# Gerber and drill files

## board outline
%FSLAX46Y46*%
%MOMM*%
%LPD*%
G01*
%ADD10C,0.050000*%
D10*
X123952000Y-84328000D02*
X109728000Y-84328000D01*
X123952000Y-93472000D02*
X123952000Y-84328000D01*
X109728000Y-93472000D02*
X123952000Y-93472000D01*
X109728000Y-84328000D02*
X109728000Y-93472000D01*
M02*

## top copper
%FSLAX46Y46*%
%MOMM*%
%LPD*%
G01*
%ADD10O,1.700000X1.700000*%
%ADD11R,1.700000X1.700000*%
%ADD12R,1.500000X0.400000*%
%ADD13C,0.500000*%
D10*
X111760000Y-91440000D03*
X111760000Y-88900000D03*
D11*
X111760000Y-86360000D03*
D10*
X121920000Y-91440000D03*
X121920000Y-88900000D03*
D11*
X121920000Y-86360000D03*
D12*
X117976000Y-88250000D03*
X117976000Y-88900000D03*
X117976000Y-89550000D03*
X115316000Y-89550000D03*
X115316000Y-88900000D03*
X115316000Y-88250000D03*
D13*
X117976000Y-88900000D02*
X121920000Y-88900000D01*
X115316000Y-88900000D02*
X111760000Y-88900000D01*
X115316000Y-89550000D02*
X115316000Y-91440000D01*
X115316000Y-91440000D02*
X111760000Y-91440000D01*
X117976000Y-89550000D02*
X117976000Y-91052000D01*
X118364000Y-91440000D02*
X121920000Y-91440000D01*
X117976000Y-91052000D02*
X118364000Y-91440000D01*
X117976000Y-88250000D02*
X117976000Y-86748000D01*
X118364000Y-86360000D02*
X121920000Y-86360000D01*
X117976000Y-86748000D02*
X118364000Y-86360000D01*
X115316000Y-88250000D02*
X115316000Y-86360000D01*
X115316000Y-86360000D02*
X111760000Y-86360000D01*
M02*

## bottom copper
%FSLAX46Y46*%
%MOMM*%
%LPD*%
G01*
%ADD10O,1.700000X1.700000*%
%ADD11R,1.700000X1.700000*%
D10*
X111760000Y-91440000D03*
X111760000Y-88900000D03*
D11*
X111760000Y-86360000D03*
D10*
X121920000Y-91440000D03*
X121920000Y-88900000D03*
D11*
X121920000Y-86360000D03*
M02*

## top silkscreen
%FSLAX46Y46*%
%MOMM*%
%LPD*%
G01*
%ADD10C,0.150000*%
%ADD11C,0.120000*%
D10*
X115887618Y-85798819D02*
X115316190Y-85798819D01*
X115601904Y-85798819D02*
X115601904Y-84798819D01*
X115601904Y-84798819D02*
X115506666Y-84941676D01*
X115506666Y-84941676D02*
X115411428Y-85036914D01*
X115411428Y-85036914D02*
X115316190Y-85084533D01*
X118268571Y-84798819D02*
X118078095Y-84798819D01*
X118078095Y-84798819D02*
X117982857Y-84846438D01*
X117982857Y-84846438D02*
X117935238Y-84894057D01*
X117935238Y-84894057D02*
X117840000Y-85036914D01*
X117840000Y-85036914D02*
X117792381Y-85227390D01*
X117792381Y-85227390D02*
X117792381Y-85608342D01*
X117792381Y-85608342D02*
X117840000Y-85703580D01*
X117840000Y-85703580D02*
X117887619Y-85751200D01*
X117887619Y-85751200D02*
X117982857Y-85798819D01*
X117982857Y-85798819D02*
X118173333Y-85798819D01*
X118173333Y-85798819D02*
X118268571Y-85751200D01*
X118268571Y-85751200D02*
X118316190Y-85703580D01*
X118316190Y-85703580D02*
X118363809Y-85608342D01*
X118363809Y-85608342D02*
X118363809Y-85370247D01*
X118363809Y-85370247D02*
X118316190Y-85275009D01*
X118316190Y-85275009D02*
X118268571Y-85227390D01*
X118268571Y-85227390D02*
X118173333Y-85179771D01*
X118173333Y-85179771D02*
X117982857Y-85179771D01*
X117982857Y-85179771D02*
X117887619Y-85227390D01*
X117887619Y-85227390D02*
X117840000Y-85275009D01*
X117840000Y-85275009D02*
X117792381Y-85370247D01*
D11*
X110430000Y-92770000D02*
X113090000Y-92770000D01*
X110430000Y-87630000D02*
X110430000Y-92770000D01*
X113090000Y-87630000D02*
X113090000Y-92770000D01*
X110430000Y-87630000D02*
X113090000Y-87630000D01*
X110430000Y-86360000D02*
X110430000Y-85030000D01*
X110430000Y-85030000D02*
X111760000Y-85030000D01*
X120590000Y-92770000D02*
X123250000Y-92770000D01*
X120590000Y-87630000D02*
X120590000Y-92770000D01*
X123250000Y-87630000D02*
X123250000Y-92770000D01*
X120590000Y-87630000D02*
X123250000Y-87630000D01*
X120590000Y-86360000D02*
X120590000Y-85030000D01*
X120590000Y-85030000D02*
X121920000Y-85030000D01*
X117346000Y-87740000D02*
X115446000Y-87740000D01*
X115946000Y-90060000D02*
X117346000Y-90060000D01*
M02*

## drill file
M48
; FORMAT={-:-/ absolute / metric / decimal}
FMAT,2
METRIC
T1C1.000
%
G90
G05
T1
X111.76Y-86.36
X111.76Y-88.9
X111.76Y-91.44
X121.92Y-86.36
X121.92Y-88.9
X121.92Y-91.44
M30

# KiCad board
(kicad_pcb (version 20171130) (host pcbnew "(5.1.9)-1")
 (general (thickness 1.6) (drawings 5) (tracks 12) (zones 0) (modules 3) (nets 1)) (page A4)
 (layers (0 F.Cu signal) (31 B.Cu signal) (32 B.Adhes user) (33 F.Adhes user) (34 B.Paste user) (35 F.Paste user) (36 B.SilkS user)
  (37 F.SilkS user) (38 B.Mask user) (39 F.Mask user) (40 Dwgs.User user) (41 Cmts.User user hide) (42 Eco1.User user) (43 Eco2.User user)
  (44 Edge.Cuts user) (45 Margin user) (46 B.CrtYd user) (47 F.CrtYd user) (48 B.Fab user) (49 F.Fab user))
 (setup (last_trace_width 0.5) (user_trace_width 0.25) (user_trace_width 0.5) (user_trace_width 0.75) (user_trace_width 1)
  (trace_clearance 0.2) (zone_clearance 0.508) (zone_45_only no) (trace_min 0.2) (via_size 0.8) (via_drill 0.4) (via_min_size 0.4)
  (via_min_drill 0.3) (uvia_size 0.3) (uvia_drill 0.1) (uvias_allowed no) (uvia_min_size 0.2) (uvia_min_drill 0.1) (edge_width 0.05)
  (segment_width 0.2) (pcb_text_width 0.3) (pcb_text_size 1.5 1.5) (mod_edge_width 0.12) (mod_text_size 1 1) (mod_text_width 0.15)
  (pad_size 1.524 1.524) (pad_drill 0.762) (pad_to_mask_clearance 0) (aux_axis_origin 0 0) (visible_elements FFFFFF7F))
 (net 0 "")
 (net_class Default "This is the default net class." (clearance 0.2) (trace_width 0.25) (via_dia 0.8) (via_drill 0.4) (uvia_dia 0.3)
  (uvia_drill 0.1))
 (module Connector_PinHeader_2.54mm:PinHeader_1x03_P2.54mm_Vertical (layer F.Cu) (at 111.76 86.36)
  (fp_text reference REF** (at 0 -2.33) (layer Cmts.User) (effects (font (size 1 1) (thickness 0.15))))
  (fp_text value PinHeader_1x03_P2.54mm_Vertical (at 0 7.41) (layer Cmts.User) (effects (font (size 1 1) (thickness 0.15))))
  (fp_line (start -1.33 6.41) (end 1.33 6.41) (layer F.SilkS) (width 0.12))
  (fp_line (start -1.33 1.27) (end -1.33 6.41) (layer F.SilkS) (width 0.12))
  (fp_line (start 1.33 1.27) (end 1.33 6.41) (layer F.SilkS) (width 0.12))
  (fp_line (start -1.33 1.27) (end 1.33 1.27) (layer F.SilkS) (width 0.12))
  (fp_line (start -1.33 0) (end -1.33 -1.33) (layer F.SilkS) (width 0.12))
  (fp_line (start -1.33 -1.33) (end 0 -1.33) (layer F.SilkS) (width 0.12))
  (pad 3 thru_hole oval (at 0 5.08) (size 1.7 1.7) (drill 1) (layers *.Cu *.Mask))
  (pad 2 thru_hole oval (at 0 2.54) (size 1.7 1.7) (drill 1) (layers *.Cu *.Mask))
  (pad 1 thru_hole rect (at 0 0) (size 1.7 1.7) (drill 1) (layers *.Cu *.Mask)))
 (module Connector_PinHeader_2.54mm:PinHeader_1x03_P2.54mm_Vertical (layer F.Cu) (at 121.92 86.36)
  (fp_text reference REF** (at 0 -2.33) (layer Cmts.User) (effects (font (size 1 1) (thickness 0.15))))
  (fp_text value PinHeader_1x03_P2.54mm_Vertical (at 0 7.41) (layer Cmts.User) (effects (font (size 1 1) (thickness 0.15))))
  (fp_line (start -1.33 6.41) (end 1.33 6.41) (layer F.SilkS) (width 0.12))
  (fp_line (start -1.33 1.27) (end -1.33 6.41) (layer F.SilkS) (width 0.12))
  (fp_line (start 1.33 1.27) (end 1.33 6.41) (layer F.SilkS) (width 0.12))
  (fp_line (start -1.33 1.27) (end 1.33 1.27) (layer F.SilkS) (width 0.12))
  (fp_line (start -1.33 0) (end -1.33 -1.33) (layer F.SilkS) (width 0.12))
  (fp_line (start -1.33 -1.33) (end 0 -1.33) (layer F.SilkS) (width 0.12))
  (pad 3 thru_hole oval (at 0 5.08) (size 1.7 1.7) (drill 1) (layers *.Cu *.Mask))
  (pad 2 thru_hole oval (at 0 2.54) (size 1.7 1.7) (drill 1) (layers *.Cu *.Mask))
  (pad 1 thru_hole rect (at 0 0) (size 1.7 1.7) (drill 1) (layers *.Cu *.Mask)))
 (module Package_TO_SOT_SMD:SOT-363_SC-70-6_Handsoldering (layer F.Cu) (at 116.646 88.9)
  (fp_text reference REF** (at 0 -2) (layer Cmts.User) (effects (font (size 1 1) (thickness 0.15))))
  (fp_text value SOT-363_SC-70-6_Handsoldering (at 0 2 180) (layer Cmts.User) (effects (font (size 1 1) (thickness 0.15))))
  (fp_line (start 0.7 -1.16) (end -1.2 -1.16) (layer F.SilkS) (width 0.12))
  (fp_line (start -0.7 1.16) (end 0.7 1.16) (layer F.SilkS) (width 0.12))
  (pad 6 smd rect (at 1.33 -0.65) (size 1.5 0.4) (layers F.Cu F.Paste F.Mask))
  (pad 5 smd rect (at 1.33 0) (size 1.5 0.4) (layers F.Cu F.Paste F.Mask))
  (pad 4 smd rect (at 1.33 0.65) (size 1.5 0.4) (layers F.Cu F.Paste F.Mask))
  (pad 3 smd rect (at -1.33 0.65) (size 1.5 0.4) (layers F.Cu F.Paste F.Mask))
  (pad 2 smd rect (at -1.33 0) (size 1.5 0.4) (layers F.Cu F.Paste F.Mask))
  (pad 1 smd rect (at -1.33 -0.65) (size 1.5 0.4) (layers F.Cu F.Paste F.Mask)))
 (gr_line (start 123.952 84.328) (end 109.728 84.328) (layer Edge.Cuts) (width 0.05))
 (gr_line (start 123.952 93.472) (end 123.952 84.328) (layer Edge.Cuts) (width 0.05))
 (gr_line (start 109.728 93.472) (end 123.952 93.472) (layer Edge.Cuts) (width 0.05))
 (gr_line (start 109.728 84.328) (end 109.728 93.472) (layer Edge.Cuts) (width 0.05))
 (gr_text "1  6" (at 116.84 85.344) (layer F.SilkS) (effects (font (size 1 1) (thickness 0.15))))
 (segment (start 117.976 88.9) (end 121.92 88.9) (width 0.5) (layer F.Cu) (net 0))
 (segment (start 115.316 88.9) (end 111.76 88.9) (width 0.5) (layer F.Cu) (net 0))
 (segment (start 115.316 89.55) (end 115.316 91.44) (width 0.5) (layer F.Cu) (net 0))
 (segment (start 115.316 91.44) (end 111.76 91.44) (width 0.5) (layer F.Cu) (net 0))
 (segment (start 117.976 89.55) (end 117.976 91.052) (width 0.5) (layer F.Cu) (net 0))
 (segment (start 118.364 91.44) (end 121.92 91.44) (width 0.5) (layer F.Cu) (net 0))
 (segment (start 117.976 91.052) (end 118.364 91.44) (width 0.5) (layer F.Cu) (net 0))
 (segment (start 117.976 88.25) (end 117.976 86.748) (width 0.5) (layer F.Cu) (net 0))
 (segment (start 118.364 86.36) (end 121.92 86.36) (width 0.5) (layer F.Cu) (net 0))
 (segment (start 117.976 86.748) (end 118.364 86.36) (width 0.5) (layer F.Cu) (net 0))
 (segment (start 115.316 88.25) (end 115.316 86.36) (width 0.5) (layer F.Cu) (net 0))
 (segment (start 115.316 86.36) (end 111.76 86.36) (width 0.5) (layer F.Cu) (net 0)))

